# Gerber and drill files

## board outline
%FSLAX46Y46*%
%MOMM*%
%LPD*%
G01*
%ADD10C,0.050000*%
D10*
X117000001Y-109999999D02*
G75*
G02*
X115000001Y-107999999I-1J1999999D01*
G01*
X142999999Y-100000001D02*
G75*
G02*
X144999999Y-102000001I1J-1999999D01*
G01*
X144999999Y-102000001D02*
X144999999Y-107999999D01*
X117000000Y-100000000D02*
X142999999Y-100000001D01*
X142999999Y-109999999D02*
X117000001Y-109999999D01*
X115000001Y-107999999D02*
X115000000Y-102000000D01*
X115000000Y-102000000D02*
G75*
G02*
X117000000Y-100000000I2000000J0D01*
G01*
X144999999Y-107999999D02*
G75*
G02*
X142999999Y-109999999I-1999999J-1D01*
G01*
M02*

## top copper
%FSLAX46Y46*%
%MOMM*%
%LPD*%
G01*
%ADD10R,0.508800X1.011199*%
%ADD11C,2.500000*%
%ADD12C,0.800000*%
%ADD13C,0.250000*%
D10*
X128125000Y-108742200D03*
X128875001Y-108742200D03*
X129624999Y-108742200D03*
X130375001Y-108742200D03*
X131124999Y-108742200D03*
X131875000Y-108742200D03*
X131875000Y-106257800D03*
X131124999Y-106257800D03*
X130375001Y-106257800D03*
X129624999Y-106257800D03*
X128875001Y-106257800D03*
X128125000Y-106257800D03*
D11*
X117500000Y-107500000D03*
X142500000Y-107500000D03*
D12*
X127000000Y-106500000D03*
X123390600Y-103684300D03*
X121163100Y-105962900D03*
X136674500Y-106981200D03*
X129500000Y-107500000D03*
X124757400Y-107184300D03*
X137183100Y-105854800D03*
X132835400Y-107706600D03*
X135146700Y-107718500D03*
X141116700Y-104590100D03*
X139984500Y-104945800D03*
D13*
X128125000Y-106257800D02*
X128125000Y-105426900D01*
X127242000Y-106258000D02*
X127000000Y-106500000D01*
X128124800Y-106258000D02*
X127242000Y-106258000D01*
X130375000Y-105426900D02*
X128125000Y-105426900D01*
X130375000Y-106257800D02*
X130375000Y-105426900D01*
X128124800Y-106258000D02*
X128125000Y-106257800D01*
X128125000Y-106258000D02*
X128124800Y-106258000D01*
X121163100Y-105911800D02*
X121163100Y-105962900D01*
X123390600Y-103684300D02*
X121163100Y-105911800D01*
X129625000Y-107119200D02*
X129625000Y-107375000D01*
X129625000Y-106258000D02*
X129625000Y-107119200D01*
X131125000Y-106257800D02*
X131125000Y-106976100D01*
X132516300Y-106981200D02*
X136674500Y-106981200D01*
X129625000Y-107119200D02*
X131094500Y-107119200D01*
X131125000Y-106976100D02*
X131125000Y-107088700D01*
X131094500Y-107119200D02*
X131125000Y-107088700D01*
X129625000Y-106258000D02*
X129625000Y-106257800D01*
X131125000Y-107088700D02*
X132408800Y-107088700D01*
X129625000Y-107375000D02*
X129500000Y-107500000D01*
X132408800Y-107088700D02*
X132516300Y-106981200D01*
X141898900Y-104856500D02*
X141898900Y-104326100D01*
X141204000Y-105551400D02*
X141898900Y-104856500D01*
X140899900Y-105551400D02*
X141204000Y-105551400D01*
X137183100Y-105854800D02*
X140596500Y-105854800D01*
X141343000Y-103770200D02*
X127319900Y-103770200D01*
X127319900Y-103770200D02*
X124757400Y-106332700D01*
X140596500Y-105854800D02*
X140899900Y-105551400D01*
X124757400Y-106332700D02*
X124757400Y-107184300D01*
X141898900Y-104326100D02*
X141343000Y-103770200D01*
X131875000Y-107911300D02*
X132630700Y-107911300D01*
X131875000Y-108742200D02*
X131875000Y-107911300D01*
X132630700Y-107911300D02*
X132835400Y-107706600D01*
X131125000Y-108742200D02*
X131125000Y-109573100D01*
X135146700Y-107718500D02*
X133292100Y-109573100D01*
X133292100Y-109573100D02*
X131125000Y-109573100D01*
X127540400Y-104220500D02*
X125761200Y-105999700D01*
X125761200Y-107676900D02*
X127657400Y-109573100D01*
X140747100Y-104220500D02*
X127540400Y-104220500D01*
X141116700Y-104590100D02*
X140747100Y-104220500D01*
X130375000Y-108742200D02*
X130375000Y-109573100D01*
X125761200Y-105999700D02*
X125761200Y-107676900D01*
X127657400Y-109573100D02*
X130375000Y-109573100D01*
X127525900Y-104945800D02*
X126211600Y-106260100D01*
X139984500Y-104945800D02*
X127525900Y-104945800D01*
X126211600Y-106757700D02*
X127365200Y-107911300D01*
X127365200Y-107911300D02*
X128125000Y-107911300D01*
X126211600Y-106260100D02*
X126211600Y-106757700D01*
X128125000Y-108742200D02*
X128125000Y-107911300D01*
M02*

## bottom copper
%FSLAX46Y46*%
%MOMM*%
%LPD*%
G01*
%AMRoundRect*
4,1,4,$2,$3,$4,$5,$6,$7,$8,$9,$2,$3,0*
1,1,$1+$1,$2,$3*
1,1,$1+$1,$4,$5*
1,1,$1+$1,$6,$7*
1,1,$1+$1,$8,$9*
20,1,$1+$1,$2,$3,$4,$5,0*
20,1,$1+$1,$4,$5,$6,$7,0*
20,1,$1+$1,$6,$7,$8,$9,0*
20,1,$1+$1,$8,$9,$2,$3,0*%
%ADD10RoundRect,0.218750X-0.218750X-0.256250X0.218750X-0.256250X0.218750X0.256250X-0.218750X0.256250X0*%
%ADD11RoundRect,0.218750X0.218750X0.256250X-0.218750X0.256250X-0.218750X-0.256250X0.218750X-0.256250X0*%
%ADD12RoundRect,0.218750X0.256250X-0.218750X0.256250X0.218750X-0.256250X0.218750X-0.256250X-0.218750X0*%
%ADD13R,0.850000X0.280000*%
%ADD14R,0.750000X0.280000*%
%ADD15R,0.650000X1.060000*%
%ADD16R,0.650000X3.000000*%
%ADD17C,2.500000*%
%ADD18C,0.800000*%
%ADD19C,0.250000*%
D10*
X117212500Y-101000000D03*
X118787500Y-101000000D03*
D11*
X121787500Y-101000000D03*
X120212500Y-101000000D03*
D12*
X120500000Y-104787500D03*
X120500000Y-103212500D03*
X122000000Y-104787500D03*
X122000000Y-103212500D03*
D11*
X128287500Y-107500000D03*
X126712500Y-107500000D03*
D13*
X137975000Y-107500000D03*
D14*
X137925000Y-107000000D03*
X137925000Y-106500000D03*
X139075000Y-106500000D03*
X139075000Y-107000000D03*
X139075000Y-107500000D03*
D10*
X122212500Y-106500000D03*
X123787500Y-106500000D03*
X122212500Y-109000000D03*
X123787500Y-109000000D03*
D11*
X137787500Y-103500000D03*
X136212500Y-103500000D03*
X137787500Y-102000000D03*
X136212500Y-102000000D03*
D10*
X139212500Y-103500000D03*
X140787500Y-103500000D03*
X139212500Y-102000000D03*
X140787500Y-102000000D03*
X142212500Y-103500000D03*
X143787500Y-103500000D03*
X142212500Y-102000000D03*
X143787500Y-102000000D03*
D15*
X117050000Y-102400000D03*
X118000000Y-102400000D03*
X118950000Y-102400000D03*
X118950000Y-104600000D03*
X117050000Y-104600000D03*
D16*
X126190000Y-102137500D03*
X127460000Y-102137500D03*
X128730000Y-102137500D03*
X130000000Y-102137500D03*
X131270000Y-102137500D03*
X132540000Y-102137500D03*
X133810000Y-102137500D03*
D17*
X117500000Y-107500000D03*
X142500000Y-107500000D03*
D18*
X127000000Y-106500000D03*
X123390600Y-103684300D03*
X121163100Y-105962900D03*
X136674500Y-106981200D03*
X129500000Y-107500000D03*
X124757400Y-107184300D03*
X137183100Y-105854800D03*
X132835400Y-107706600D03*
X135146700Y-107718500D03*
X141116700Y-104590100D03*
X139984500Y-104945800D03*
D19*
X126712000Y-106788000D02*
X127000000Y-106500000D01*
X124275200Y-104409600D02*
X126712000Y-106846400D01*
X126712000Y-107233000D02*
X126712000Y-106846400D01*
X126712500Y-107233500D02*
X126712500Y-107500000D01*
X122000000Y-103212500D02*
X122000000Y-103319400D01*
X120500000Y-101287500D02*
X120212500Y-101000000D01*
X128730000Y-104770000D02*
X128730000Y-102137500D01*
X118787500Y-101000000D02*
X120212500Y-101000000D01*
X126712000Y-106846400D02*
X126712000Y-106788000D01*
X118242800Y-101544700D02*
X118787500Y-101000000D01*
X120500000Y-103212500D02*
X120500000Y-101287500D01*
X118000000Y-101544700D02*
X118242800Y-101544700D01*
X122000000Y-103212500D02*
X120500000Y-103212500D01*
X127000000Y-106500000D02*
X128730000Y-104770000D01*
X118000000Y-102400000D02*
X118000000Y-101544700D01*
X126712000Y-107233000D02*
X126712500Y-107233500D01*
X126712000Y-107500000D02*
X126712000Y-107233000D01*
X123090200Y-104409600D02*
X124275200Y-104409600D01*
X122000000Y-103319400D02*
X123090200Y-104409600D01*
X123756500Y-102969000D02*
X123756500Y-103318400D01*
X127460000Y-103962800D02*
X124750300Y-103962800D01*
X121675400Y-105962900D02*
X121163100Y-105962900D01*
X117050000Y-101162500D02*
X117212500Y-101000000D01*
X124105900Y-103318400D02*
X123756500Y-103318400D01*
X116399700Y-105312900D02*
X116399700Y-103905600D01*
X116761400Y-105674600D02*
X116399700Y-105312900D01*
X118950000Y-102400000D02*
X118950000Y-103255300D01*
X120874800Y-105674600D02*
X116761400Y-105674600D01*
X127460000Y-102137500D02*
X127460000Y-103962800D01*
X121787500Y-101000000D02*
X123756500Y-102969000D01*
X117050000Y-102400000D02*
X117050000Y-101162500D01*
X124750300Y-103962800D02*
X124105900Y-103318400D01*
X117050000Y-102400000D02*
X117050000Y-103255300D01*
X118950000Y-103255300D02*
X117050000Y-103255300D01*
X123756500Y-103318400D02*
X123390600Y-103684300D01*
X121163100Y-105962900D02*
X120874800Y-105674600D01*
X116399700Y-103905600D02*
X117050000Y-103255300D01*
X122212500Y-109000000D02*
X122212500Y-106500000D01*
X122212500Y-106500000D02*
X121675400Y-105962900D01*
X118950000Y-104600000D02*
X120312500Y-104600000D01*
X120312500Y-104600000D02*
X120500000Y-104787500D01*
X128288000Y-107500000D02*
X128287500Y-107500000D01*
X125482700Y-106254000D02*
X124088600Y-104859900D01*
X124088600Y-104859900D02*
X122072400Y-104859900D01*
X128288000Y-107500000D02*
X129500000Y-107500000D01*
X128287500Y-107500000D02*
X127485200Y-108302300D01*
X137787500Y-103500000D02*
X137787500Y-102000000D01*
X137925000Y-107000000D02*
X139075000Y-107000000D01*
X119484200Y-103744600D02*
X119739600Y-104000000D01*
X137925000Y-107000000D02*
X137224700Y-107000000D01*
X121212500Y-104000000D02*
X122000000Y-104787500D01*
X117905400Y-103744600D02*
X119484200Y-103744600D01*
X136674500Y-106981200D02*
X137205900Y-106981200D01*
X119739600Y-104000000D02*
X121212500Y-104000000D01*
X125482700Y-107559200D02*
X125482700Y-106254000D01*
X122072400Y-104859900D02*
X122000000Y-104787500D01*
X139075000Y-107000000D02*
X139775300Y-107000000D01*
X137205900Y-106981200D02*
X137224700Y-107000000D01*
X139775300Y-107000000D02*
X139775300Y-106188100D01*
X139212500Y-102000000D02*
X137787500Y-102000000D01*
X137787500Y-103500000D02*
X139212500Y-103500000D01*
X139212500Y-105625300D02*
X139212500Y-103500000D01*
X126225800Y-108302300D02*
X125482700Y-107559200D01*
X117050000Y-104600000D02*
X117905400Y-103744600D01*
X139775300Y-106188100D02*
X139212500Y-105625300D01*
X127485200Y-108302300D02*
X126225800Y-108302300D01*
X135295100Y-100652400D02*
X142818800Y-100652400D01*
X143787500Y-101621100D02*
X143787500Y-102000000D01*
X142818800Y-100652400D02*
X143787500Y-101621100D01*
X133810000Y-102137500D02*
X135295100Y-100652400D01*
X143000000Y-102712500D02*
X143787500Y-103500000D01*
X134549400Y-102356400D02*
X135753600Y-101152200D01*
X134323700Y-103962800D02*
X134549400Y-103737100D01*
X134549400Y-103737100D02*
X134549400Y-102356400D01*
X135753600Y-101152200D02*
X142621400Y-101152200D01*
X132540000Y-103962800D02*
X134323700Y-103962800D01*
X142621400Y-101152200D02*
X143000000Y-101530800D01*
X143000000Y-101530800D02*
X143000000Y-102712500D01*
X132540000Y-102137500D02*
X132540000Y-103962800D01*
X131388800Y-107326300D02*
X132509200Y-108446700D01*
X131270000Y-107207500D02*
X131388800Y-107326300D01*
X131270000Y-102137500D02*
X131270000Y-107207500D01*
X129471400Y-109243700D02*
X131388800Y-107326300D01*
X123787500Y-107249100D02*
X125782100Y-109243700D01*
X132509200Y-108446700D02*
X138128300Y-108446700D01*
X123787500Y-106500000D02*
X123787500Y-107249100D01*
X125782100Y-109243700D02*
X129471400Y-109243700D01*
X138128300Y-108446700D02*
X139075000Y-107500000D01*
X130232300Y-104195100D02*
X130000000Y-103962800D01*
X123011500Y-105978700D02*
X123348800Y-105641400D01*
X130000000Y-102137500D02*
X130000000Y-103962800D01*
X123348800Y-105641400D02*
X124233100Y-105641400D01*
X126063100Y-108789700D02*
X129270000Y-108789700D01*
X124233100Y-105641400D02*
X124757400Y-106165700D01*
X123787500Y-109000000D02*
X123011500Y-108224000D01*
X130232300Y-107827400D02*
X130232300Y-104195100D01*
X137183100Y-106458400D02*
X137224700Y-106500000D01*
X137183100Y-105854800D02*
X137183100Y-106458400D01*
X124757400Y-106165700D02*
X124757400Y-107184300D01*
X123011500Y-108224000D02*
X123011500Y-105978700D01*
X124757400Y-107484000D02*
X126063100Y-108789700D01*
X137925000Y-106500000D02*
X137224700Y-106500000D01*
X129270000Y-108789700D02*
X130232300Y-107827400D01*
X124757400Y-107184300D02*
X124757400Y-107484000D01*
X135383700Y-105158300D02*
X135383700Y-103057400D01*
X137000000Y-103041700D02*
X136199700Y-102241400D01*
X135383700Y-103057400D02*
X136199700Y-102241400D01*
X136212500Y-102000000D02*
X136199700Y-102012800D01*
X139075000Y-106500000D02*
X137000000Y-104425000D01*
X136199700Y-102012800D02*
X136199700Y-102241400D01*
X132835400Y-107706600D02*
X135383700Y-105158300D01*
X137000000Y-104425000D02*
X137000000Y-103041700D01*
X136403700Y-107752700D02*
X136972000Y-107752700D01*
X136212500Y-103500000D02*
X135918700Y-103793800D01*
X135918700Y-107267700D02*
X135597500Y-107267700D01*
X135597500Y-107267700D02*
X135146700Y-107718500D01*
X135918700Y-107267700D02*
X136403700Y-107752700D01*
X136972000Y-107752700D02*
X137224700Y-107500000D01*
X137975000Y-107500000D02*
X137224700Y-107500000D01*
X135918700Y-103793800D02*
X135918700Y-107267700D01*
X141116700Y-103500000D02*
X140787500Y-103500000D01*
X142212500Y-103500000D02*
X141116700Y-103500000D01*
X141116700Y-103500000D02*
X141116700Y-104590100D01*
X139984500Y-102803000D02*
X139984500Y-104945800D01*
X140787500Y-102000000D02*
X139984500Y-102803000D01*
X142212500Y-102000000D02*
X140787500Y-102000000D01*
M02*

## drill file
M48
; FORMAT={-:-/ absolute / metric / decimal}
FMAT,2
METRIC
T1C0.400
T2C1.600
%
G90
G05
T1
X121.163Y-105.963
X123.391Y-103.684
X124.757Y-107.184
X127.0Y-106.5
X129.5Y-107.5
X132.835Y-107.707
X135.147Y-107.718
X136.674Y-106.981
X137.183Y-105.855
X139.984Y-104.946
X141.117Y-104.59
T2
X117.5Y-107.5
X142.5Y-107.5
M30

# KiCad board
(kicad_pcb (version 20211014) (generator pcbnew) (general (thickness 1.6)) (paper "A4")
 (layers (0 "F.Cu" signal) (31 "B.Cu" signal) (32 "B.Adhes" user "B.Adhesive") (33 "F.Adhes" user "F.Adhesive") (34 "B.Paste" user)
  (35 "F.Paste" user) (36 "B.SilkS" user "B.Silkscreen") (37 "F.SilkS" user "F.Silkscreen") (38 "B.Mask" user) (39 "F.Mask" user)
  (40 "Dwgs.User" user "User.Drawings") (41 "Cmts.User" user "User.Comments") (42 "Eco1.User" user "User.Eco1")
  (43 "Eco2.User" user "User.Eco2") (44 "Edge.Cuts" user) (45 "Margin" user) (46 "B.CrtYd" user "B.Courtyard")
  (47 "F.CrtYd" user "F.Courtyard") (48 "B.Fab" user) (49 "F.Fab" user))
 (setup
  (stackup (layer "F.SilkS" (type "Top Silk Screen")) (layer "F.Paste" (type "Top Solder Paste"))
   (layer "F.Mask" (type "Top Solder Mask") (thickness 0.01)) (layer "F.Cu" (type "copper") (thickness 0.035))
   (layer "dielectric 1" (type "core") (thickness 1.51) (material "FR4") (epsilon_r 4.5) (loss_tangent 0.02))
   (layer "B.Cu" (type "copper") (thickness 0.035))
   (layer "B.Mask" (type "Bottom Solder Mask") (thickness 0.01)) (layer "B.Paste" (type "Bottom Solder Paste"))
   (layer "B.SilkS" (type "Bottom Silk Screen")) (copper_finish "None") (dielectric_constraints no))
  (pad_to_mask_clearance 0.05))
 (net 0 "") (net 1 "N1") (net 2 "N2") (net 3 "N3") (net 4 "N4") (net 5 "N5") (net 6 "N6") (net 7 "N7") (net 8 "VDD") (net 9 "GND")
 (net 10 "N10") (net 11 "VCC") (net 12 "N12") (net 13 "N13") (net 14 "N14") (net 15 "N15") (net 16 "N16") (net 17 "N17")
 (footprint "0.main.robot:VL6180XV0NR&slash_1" (layer "F.Cu") (at 130 107.5 90)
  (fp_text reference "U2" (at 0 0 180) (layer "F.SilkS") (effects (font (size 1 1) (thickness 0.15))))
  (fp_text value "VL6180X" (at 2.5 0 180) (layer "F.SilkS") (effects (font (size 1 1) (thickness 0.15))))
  (pad "1" smd rect locked (at -1.2422 -1.875 90) (size 1.011199 0.5088) (layers "F.Cu" "F.Paste" "F.Mask") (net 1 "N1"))
  (pad "2" smd rect locked (at -1.2422 -1.124999 90) (size 1.011199 0.5088) (layers "F.Cu" "F.Paste" "F.Mask") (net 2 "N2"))
  (pad "3" smd rect locked (at -1.2422 -0.375001 90) (size 1.011199 0.5088) (layers "F.Cu" "F.Paste" "F.Mask") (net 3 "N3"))
  (pad "4" smd rect locked (at -1.2422 0.375001 90) (size 1.011199 0.5088) (layers "F.Cu" "F.Paste" "F.Mask") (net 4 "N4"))
  (pad "5" smd rect locked (at -1.2422 1.124999 90) (size 1.011199 0.5088) (layers "F.Cu" "F.Paste" "F.Mask") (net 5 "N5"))
  (pad "6" smd rect locked (at -1.2422 1.875 90) (size 1.011199 0.5088) (layers "F.Cu" "F.Paste" "F.Mask") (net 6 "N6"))
  (pad "7" smd rect locked (at 1.2422 1.875 90) (size 1.011199 0.5088) (layers "F.Cu" "F.Paste" "F.Mask") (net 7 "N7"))
  (pad "8" smd rect locked (at 1.2422 1.124999 90) (size 1.011199 0.5088) (layers "F.Cu" "F.Paste" "F.Mask") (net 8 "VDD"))
  (pad "9" smd rect locked (at 1.2422 0.375001 90) (size 1.011199 0.5088) (layers "F.Cu" "F.Paste" "F.Mask") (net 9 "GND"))
  (pad "10" smd rect locked (at 1.2422 -0.375001 90) (size 1.011199 0.5088) (layers "F.Cu" "F.Paste" "F.Mask") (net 8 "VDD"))
  (pad "11" smd rect locked (at 1.2422 -1.124999 90) (size 1.011199 0.5088) (layers "F.Cu" "F.Paste" "F.Mask") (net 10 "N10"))
  (pad "12" smd rect locked (at 1.2422 -1.875 90) (size 1.011199 0.5088) (layers "F.Cu" "F.Paste" "F.Mask") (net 9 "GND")))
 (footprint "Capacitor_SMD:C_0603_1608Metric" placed (layer "B.Cu") (at 118 101)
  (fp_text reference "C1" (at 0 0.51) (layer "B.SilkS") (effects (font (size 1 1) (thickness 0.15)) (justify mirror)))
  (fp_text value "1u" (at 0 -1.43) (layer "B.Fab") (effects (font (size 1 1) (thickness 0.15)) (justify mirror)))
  (pad "1" smd roundrect locked (at -0.7875 0) (size 0.875 0.95) (layers "B.Cu" "B.Paste" "B.Mask") (roundrect_rratio 0.25) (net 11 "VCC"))
  (pad "2" smd roundrect locked (at 0.7875 0) (size 0.875 0.95) (layers "B.Cu" "B.Paste" "B.Mask") (roundrect_rratio 0.25) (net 9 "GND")))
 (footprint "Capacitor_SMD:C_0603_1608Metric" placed (layer "B.Cu") (at 121 101 180)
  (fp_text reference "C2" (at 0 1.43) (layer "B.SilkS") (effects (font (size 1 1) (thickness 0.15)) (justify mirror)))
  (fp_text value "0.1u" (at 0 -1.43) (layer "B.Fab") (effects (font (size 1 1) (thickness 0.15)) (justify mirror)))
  (pad "1" smd roundrect locked (at -0.7875 0 180) (size 0.875 0.95) (layers "B.Cu" "B.Paste" "B.Mask") (roundrect_rratio 0.25)
   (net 11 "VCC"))
  (pad "2" smd roundrect locked (at 0.7875 0 180) (size 0.875 0.95) (layers "B.Cu" "B.Paste" "B.Mask") (roundrect_rratio 0.25) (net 9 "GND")))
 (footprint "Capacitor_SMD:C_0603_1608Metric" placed (layer "B.Cu") (at 120.5 104 90)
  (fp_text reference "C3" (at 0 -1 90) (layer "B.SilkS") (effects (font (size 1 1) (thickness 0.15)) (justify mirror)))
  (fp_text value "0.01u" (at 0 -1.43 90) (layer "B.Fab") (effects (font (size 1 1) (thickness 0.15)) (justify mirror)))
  (pad "1" smd roundrect locked (at -0.7875 0 90) (size 0.875 0.95) (layers "B.Cu" "B.Paste" "B.Mask") (roundrect_rratio 0.25)
   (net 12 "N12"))
  (pad "2" smd roundrect locked (at 0.7875 0 90) (size 0.875 0.95) (layers "B.Cu" "B.Paste" "B.Mask") (roundrect_rratio 0.25) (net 9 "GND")))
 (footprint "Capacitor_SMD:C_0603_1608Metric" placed (layer "B.Cu") (at 122 104 90)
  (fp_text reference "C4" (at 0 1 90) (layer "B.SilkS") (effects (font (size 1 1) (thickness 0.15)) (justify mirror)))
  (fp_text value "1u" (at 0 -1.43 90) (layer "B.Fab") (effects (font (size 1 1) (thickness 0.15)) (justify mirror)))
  (pad "1" smd roundrect locked (at -0.7875 0 90) (size 0.875 0.95) (layers "B.Cu" "B.Paste" "B.Mask") (roundrect_rratio 0.25) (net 8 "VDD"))
  (pad "2" smd roundrect locked (at 0.7875 0 90) (size 0.875 0.95) (layers "B.Cu" "B.Paste" "B.Mask") (roundrect_rratio 0.25) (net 9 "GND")))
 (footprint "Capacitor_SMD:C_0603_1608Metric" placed (layer "B.Cu") (at 127.5 107.5 180)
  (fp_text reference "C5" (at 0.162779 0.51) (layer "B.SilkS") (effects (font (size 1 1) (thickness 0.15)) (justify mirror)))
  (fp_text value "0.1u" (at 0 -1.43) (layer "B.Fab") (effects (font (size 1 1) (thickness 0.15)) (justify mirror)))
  (pad "1" smd roundrect locked (at -0.7875 0 180) (size 0.875 0.95) (layers "B.Cu" "B.Paste" "B.Mask") (roundrect_rratio 0.25)
   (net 8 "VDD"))
  (pad "2" smd roundrect locked (at 0.7875 0 180) (size 0.875 0.95) (layers "B.Cu" "B.Paste" "B.Mask") (roundrect_rratio 0.25) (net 9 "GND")))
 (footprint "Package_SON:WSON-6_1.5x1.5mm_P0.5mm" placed (layer "B.Cu") (at 138.5 107)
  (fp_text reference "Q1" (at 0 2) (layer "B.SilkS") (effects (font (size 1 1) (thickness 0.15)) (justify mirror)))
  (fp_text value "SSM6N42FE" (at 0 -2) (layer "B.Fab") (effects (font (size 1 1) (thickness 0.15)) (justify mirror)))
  (pad "1" smd rect locked (at -0.525 0.5 90) (size 0.28 0.85) (layers "B.Cu" "B.Paste" "B.Mask") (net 5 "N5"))
  (pad "2" smd rect locked (at -0.575 0 90) (size 0.28 0.75) (layers "B.Cu" "B.Paste" "B.Mask") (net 8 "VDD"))
  (pad "3" smd rect locked (at -0.575 -0.5 90) (size 0.28 0.75) (layers "B.Cu" "B.Paste" "B.Mask") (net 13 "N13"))
  (pad "4" smd rect locked (at 0.575 -0.5 90) (size 0.28 0.75) (layers "B.Cu" "B.Paste" "B.Mask") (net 6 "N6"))
  (pad "5" smd rect locked (at 0.575 0 90) (size 0.28 0.75) (layers "B.Cu" "B.Paste" "B.Mask") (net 8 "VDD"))
  (pad "6" smd rect locked (at 0.575 0.5 90) (size 0.28 0.75) (layers "B.Cu" "B.Paste" "B.Mask") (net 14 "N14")))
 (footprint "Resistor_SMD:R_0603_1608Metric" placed (layer "B.Cu") (at 123 106.5)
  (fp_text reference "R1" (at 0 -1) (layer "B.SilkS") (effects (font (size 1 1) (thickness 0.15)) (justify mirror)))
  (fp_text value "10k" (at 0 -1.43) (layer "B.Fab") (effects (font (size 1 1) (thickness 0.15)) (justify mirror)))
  (pad "1" smd roundrect locked (at -0.7875 0) (size 0.875 0.95) (layers "B.Cu" "B.Paste" "B.Mask") (roundrect_rratio 0.25) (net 11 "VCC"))
  (pad "2" smd roundrect locked (at 0.7875 0) (size 0.875 0.95) (layers "B.Cu" "B.Paste" "B.Mask") (roundrect_rratio 0.25) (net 14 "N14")))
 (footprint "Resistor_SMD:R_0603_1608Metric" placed (layer "B.Cu") (at 123 109)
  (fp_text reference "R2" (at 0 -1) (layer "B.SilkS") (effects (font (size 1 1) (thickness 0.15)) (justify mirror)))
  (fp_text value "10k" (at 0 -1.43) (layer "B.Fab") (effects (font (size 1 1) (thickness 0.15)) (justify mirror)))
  (pad "1" smd roundrect locked (at -0.7875 0) (size 0.875 0.95) (layers "B.Cu" "B.Paste" "B.Mask") (roundrect_rratio 0.25) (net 11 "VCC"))
  (pad "2" smd roundrect locked (at 0.7875 0) (size 0.875 0.95) (layers "B.Cu" "B.Paste" "B.Mask") (roundrect_rratio 0.25) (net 13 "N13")))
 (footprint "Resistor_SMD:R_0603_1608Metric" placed (layer "B.Cu") (at 137 103.5 180)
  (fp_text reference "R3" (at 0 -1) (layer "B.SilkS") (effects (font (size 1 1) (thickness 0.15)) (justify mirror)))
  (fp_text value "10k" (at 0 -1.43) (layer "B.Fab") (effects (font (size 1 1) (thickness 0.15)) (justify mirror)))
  (pad "1" smd roundrect locked (at -0.7875 0 180) (size 0.875 0.95) (layers "B.Cu" "B.Paste" "B.Mask") (roundrect_rratio 0.25)
   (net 8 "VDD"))
  (pad "2" smd roundrect locked (at 0.7875 0 180) (size 0.875 0.95) (layers "B.Cu" "B.Paste" "B.Mask") (roundrect_rratio 0.25) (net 5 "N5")))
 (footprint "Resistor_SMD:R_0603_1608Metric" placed (layer "B.Cu") (at 137 102 180)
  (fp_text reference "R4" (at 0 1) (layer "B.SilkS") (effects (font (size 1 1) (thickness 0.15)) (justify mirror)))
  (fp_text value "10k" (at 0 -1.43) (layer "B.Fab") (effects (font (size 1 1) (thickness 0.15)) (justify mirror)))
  (pad "1" smd roundrect locked (at -0.7875 0 180) (size 0.875 0.95) (layers "B.Cu" "B.Paste" "B.Mask") (roundrect_rratio 0.25)
   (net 8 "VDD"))
  (pad "2" smd roundrect locked (at 0.7875 0 180) (size 0.875 0.95) (layers "B.Cu" "B.Paste" "B.Mask") (roundrect_rratio 0.25) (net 6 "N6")))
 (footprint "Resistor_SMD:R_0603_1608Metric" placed (layer "B.Cu") (at 140 103.5)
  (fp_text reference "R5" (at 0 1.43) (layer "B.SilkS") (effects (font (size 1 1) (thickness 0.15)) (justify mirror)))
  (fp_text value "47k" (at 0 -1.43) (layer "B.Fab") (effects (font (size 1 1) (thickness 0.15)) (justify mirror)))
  (pad "1" smd roundrect locked (at -0.7875 0) (size 0.875 0.95) (layers "B.Cu" "B.Paste" "B.Mask") (roundrect_rratio 0.25) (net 8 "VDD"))
  (pad "2" smd roundrect locked (at 0.7875 0) (size 0.875 0.95) (layers "B.Cu" "B.Paste" "B.Mask") (roundrect_rratio 0.25) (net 4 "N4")))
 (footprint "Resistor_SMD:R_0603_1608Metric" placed (layer "B.Cu") (at 140 102)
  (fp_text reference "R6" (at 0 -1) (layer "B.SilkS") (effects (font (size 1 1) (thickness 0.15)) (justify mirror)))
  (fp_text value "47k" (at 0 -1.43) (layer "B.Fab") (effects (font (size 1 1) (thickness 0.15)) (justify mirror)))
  (pad "1" smd roundrect locked (at -0.7875 0) (size 0.875 0.95) (layers "B.Cu" "B.Paste" "B.Mask") (roundrect_rratio 0.25) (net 8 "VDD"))
  (pad "2" smd roundrect locked (at 0.7875 0) (size 0.875 0.95) (layers "B.Cu" "B.Paste" "B.Mask") (roundrect_rratio 0.25) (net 1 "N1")))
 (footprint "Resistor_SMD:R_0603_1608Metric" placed (layer "B.Cu") (at 143 103.5)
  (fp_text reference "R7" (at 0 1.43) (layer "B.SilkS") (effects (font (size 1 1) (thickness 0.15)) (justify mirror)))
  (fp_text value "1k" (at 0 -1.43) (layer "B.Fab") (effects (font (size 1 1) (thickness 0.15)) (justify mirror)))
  (pad "1" smd roundrect locked (at -0.7875 0) (size 0.875 0.95) (layers "B.Cu" "B.Paste" "B.Mask") (roundrect_rratio 0.25) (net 4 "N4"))
  (pad "2" smd roundrect locked (at 0.7875 0) (size 0.875 0.95) (layers "B.Cu" "B.Paste" "B.Mask") (roundrect_rratio 0.25) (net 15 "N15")))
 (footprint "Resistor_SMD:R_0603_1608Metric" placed (layer "B.Cu") (at 143 102)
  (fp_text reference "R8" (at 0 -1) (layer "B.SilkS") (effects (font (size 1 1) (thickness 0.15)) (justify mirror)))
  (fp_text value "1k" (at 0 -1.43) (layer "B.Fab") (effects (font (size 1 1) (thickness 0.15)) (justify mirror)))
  (pad "1" smd roundrect locked (at -0.7875 0) (size 0.875 0.95) (layers "B.Cu" "B.Paste" "B.Mask") (roundrect_rratio 0.25) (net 1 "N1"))
  (pad "2" smd roundrect locked (at 0.7875 0) (size 0.875 0.95) (layers "B.Cu" "B.Paste" "B.Mask") (roundrect_rratio 0.25) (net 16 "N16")))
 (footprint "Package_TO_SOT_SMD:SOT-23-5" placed (layer "B.Cu") (at 118 103.5 -90)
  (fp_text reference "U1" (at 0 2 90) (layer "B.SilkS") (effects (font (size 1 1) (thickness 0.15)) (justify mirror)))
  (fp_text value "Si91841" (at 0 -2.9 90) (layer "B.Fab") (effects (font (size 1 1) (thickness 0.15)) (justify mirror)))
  (pad "1" smd rect locked (at -1.1 0.95 270) (size 1.06 0.65) (layers "B.Cu" "B.Paste" "B.Mask") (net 11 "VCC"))
  (pad "2" smd rect locked (at -1.1 0 270) (size 1.06 0.65) (layers "B.Cu" "B.Paste" "B.Mask") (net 9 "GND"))
  (pad "3" smd rect locked (at -1.1 -0.95 270) (size 1.06 0.65) (layers "B.Cu" "B.Paste" "B.Mask") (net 11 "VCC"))
  (pad "4" smd rect locked (at 1.1 -0.95 270) (size 1.06 0.65) (layers "B.Cu" "B.Paste" "B.Mask") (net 12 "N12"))
  (pad "5" smd rect locked (at 1.1 0.95 270) (size 1.06 0.65) (layers "B.Cu" "B.Paste" "B.Mask") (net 8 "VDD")))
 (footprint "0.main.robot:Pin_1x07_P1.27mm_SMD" (layer "B.Cu") (at 130 103.6375 -90)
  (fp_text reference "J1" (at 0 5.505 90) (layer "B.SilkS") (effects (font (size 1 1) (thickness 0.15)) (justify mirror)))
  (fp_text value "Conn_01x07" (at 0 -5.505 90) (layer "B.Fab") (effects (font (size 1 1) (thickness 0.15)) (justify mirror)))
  (pad "1" smd rect locked (at -1.5 3.81 270) (size 3 0.65) (layers "B.Cu" "B.Paste" "B.Mask") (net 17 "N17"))
  (pad "2" smd rect locked (at -1.5 2.54 270) (size 3 0.65) (layers "B.Cu" "B.Paste" "B.Mask") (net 11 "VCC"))
  (pad "3" smd rect locked (at -1.5 1.27 270) (size 3 0.65) (layers "B.Cu" "B.Paste" "B.Mask") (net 9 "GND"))
  (pad "4" smd rect locked (at -1.5 0 270) (size 3 0.65) (layers "B.Cu" "B.Paste" "B.Mask") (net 13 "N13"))
  (pad "5" smd rect locked (at -1.5 -1.27 270) (size 3 0.65) (layers "B.Cu" "B.Paste" "B.Mask") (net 14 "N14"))
  (pad "6" smd rect locked (at -1.5 -2.54 270) (size 3 0.65) (layers "B.Cu" "B.Paste" "B.Mask") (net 15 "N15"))
  (pad "7" smd rect locked (at -1.5 -3.81 270) (size 3 0.65) (layers "B.Cu" "B.Paste" "B.Mask") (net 16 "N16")))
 (gr_arc (start 117.000001 109.999999) (mid 115.585787 109.414213) (end 115.000001 107.999999) (layer "Edge.Cuts") (width 0.05))
 (gr_arc (start 142.999999 100.000001) (mid 144.414213 100.585787) (end 144.999999 102.000001) (layer "Edge.Cuts") (width 0.05))
 (gr_line (start 144.999999 102.000001) (end 144.999999 107.999999) (layer "Edge.Cuts") (width 0.05))
 (gr_line (start 117 100) (end 142.999999 100.000001) (layer "Edge.Cuts") (width 0.05))
 (gr_line (start 142.999999 109.999999) (end 117.000001 109.999999) (layer "Edge.Cuts") (width 0.05))
 (gr_line (start 115.000001 107.999999) (end 115 102) (layer "Edge.Cuts") (width 0.05))
 (gr_arc (start 115 102) (mid 115.585786 100.585786) (end 117 100) (layer "Edge.Cuts") (width 0.05))
 (gr_arc (start 144.999999 107.999999) (mid 144.414213 109.414213) (end 142.999999 109.999999) (layer "Edge.Cuts") (width 0.05))
 (via (at 117.5 107.5) (size 2.5) (drill 1.6) (layers "F.Cu" "B.Cu") (free) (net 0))
 (via (at 142.5 107.5) (size 2.5) (drill 1.6) (layers "F.Cu" "B.Cu") (free) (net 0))
 (segment (start 128.125 106.2578) (end 128.125 105.4269) (width 0.25) (layer "F.Cu") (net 9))
 (segment (start 127.242 106.258) (end 127 106.5) (width 0.25) (layer "F.Cu") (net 9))
 (segment (start 128.1248 106.258) (end 127.242 106.258) (width 0.25) (layer "F.Cu") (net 9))
 (segment (start 130.375 105.4269) (end 128.125 105.4269) (width 0.25) (layer "F.Cu") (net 9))
 (segment (start 130.375 106.2578) (end 130.375 105.4269) (width 0.25) (layer "F.Cu") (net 9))
 (segment (start 128.1248 106.258) (end 128.125 106.2578) (width 0.25) (layer "F.Cu") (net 9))
 (segment (start 128.125 106.258) (end 128.1248 106.258) (width 0.25) (layer "F.Cu") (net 9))
 (via (at 127 106.5) (size 0.8) (drill 0.4) (layers "F.Cu" "B.Cu") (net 9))
 (segment (start 126.712 106.788) (end 127 106.5) (width 0.25) (layer "B.Cu") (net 9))
 (segment (start 124.2752 104.4096) (end 126.712 106.8464) (width 0.25) (layer "B.Cu") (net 9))
 (segment (start 126.712 107.233) (end 126.712 106.8464) (width 0.25) (layer "B.Cu") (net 9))
 (segment (start 126.7125 107.2335) (end 126.7125 107.5) (width 0.25) (layer "B.Cu") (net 9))
 (segment (start 122 103.2125) (end 122 103.3194) (width 0.25) (layer "B.Cu") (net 9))
 (segment (start 120.5 101.2875) (end 120.2125 101) (width 0.25) (layer "B.Cu") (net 9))
 (segment (start 128.73 104.77) (end 128.73 102.1375) (width 0.25) (layer "B.Cu") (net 9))
 (segment (start 118.7875 101) (end 120.2125 101) (width 0.25) (layer "B.Cu") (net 9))
 (segment (start 126.712 106.8464) (end 126.712 106.788) (width 0.25) (layer "B.Cu") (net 9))
 (segment (start 118.2428 101.5447) (end 118.7875 101) (width 0.25) (layer "B.Cu") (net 9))
 (segment (start 120.5 103.2125) (end 120.5 101.2875) (width 0.25) (layer "B.Cu") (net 9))
 (segment (start 118 101.5447) (end 118.2428 101.5447) (width 0.25) (layer "B.Cu") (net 9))
 (segment (start 122 103.2125) (end 120.5 103.2125) (width 0.25) (layer "B.Cu") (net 9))
 (segment (start 127 106.5) (end 128.73 104.77) (width 0.25) (layer "B.Cu") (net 9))
 (segment (start 118 102.4) (end 118 101.5447) (width 0.25) (layer "B.Cu") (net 9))
 (segment (start 126.712 107.233) (end 126.7125 107.2335) (width 0.25) (layer "B.Cu") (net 9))
 (segment (start 126.712 107.5) (end 126.712 107.233) (width 0.25) (layer "B.Cu") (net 9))
 (segment (start 123.0902 104.4096) (end 124.2752 104.4096) (width 0.25) (layer "B.Cu") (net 9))
 (segment (start 122 103.3194) (end 123.0902 104.4096) (width 0.25) (layer "B.Cu") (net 9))
 (segment (start 121.1631 105.9118) (end 121.1631 105.9629) (width 0.25) (layer "F.Cu") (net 11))
 (segment (start 123.3906 103.6843) (end 121.1631 105.9118) (width 0.25) (layer "F.Cu") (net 11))
 (via (at 123.3906 103.6843) (size 0.8) (drill 0.4) (layers "F.Cu" "B.Cu") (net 11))
 (via (at 121.1631 105.9629) (size 0.8) (drill 0.4) (layers "F.Cu" "B.Cu") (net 11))
 (segment (start 123.7565 102.969) (end 123.7565 103.3184) (width 0.25) (layer "B.Cu") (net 11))
 (segment (start 127.46 103.9628) (end 124.7503 103.9628) (width 0.25) (layer "B.Cu") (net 11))
 (segment (start 121.6754 105.9629) (end 121.1631 105.9629) (width 0.25) (layer "B.Cu") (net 11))
 (segment (start 117.05 101.1625) (end 117.2125 101) (width 0.25) (layer "B.Cu") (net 11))
 (segment (start 124.1059 103.3184) (end 123.7565 103.3184) (width 0.25) (layer "B.Cu") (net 11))
 (segment (start 116.3997 105.3129) (end 116.3997 103.9056) (width 0.25) (layer "B.Cu") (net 11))
 (segment (start 116.7614 105.6746) (end 116.3997 105.3129) (width 0.25) (layer "B.Cu") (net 11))
 (segment (start 118.95 102.4) (end 118.95 103.2553) (width 0.25) (layer "B.Cu") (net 11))
 (segment (start 120.8748 105.6746) (end 116.7614 105.6746) (width 0.25) (layer "B.Cu") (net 11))
 (segment (start 127.46 102.1375) (end 127.46 103.9628) (width 0.25) (layer "B.Cu") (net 11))
 (segment (start 121.7875 101) (end 123.7565 102.969) (width 0.25) (layer "B.Cu") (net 11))
 (segment (start 117.05 102.4) (end 117.05 101.1625) (width 0.25) (layer "B.Cu") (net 11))
 (segment (start 124.7503 103.9628) (end 124.1059 103.3184) (width 0.25) (layer "B.Cu") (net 11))
 (segment (start 117.05 102.4) (end 117.05 103.2553) (width 0.25) (layer "B.Cu") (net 11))
 (segment (start 118.95 103.2553) (end 117.05 103.2553) (width 0.25) (layer "B.Cu") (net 11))
 (segment (start 123.7565 103.3184) (end 123.3906 103.6843) (width 0.25) (layer "B.Cu") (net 11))
 (segment (start 121.1631 105.9629) (end 120.8748 105.6746) (width 0.25) (layer "B.Cu") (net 11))
 (segment (start 116.3997 103.9056) (end 117.05 103.2553) (width 0.25) (layer "B.Cu") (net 11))
 (segment (start 122.2125 109) (end 122.2125 106.5) (width 0.25) (layer "B.Cu") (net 11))
 (segment (start 122.2125 106.5) (end 121.6754 105.9629) (width 0.25) (layer "B.Cu") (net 11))
 (segment (start 118.95 104.6) (end 120.3125 104.6) (width 0.25) (layer "B.Cu") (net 12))
 (segment (start 120.3125 104.6) (end 120.5 104.7875) (width 0.25) (layer "B.Cu") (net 12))
 (segment (start 129.625 107.1192) (end 129.625 107.375) (width 0.25) (layer "F.Cu") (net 8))
 (segment (start 129.625 106.258) (end 129.625 107.1192) (width 0.25) (layer "F.Cu") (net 8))
 (segment (start 131.125 106.2578) (end 131.125 106.9761) (width 0.25) (layer "F.Cu") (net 8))
 (segment (start 132.5163 106.9812) (end 136.6745 106.9812) (width 0.25) (layer "F.Cu") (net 8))
 (segment (start 129.625 107.1192) (end 131.0945 107.1192) (width 0.25) (layer "F.Cu") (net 8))
 (segment (start 131.125 106.9761) (end 131.125 107.0887) (width 0.25) (layer "F.Cu") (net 8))
 (segment (start 131.0945 107.1192) (end 131.125 107.0887) (width 0.25) (layer "F.Cu") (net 8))
 (segment (start 129.625 106.258) (end 129.625 106.2578) (width 0.25) (layer "F.Cu") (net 8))
 (segment (start 131.125 107.0887) (end 132.4088 107.0887) (width 0.25) (layer "F.Cu") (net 8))
 (segment (start 129.625 107.375) (end 129.5 107.5) (width 0.25) (layer "F.Cu") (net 8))
 (segment (start 132.4088 107.0887) (end 132.5163 106.9812) (width 0.25) (layer "F.Cu") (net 8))
 (via (at 136.6745 106.9812) (size 0.8) (drill 0.4) (layers "F.Cu" "B.Cu") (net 8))
 (via (at 129.5 107.5) (size 0.8) (drill 0.4) (layers "F.Cu" "B.Cu") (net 8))
 (segment (start 128.288 107.5) (end 128.2875 107.5) (width 0.25) (layer "B.Cu") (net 8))
 (segment (start 125.4827 106.254) (end 124.0886 104.8599) (width 0.25) (layer "B.Cu") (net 8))
 (segment (start 124.0886 104.8599) (end 122.0724 104.8599) (width 0.25) (layer "B.Cu") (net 8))
 (segment (start 128.288 107.5) (end 129.5 107.5) (width 0.25) (layer "B.Cu") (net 8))
 (segment (start 128.2875 107.5) (end 127.4852 108.3023) (width 0.25) (layer "B.Cu") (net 8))
 (segment (start 137.7875 103.5) (end 137.7875 102) (width 0.25) (layer "B.Cu") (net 8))
 (segment (start 137.925 107) (end 139.075 107) (width 0.25) (layer "B.Cu") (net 8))
 (segment (start 119.4842 103.7446) (end 119.7396 104) (width 0.25) (layer "B.Cu") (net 8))
 (segment (start 137.925 107) (end 137.2247 107) (width 0.25) (layer "B.Cu") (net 8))
 (segment (start 121.2125 104) (end 122 104.7875) (width 0.25) (layer "B.Cu") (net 8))
 (segment (start 117.9054 103.7446) (end 119.4842 103.7446) (width 0.25) (layer "B.Cu") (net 8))
 (segment (start 136.6745 106.9812) (end 137.2059 106.9812) (width 0.25) (layer "B.Cu") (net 8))
 (segment (start 119.7396 104) (end 121.2125 104) (width 0.25) (layer "B.Cu") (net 8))
 (segment (start 125.4827 107.5592) (end 125.4827 106.254) (width 0.25) (layer "B.Cu") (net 8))
 (segment (start 122.0724 104.8599) (end 122 104.7875) (width 0.25) (layer "B.Cu") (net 8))
 (segment (start 139.075 107) (end 139.7753 107) (width 0.25) (layer "B.Cu") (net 8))
 (segment (start 137.2059 106.9812) (end 137.2247 107) (width 0.25) (layer "B.Cu") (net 8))
 (segment (start 139.7753 107) (end 139.7753 106.1881) (width 0.25) (layer "B.Cu") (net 8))
 (segment (start 139.2125 102) (end 137.7875 102) (width 0.25) (layer "B.Cu") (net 8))
 (segment (start 137.7875 103.5) (end 139.2125 103.5) (width 0.25) (layer "B.Cu") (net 8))
 (segment (start 139.2125 105.6253) (end 139.2125 103.5) (width 0.25) (layer "B.Cu") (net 8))
 (segment (start 126.2258 108.3023) (end 125.4827 107.5592) (width 0.25) (layer "B.Cu") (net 8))
 (segment (start 117.05 104.6) (end 117.9054 103.7446) (width 0.25) (layer "B.Cu") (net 8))
 (segment (start 139.7753 106.1881) (end 139.2125 105.6253) (width 0.25) (layer "B.Cu") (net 8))
 (segment (start 127.4852 108.3023) (end 126.2258 108.3023) (width 0.25) (layer "B.Cu") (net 8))
 (segment (start 135.2951 100.6524) (end 142.8188 100.6524) (width 0.25) (layer "B.Cu") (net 16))
 (segment (start 143.7875 101.6211) (end 143.7875 102) (width 0.25) (layer "B.Cu") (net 16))
 (segment (start 142.8188 100.6524) (end 143.7875 101.6211) (width 0.25) (layer "B.Cu") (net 16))
 (segment (start 133.81 102.1375) (end 135.2951 100.6524) (width 0.25) (layer "B.Cu") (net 16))
 (segment (start 143 102.7125) (end 143.7875 103.5) (width 0.25) (layer "B.Cu") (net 15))
 (segment (start 134.5494 102.3564) (end 135.7536 101.1522) (width 0.25) (layer "B.Cu") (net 15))
 (segment (start 134.3237 103.9628) (end 134.5494 103.7371) (width 0.25) (layer "B.Cu") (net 15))
 (segment (start 134.5494 103.7371) (end 134.5494 102.3564) (width 0.25) (layer "B.Cu") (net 15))
 (segment (start 135.7536 101.1522) (end 142.6214 101.1522) (width 0.25) (layer "B.Cu") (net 15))
 (segment (start 132.54 103.9628) (end 134.3237 103.9628) (width 0.25) (layer "B.Cu") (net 15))
 (segment (start 142.6214 101.1522) (end 143 101.5308) (width 0.25) (layer "B.Cu") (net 15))
 (segment (start 143 101.5308) (end 143 102.7125) (width 0.25) (layer "B.Cu") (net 15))
 (segment (start 132.54 102.1375) (end 132.54 103.9628) (width 0.25) (layer "B.Cu") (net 15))
 (segment (start 131.3888 107.3263) (end 132.5092 108.4467) (width 0.25) (layer "B.Cu") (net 14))
 (segment (start 131.27 107.2075) (end 131.3888 107.3263) (width 0.25) (layer "B.Cu") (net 14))
 (segment (start 131.27 102.1375) (end 131.27 107.2075) (width 0.25) (layer "B.Cu") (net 14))
 (segment (start 129.4714 109.2437) (end 131.3888 107.3263) (width 0.25) (layer "B.Cu") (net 14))
 (segment (start 123.7875 107.2491) (end 125.7821 109.2437) (width 0.25) (layer "B.Cu") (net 14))
 (segment (start 132.5092 108.4467) (end 138.1283 108.4467) (width 0.25) (layer "B.Cu") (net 14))
 (segment (start 123.7875 106.5) (end 123.7875 107.2491) (width 0.25) (layer "B.Cu") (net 14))
 (segment (start 125.7821 109.2437) (end 129.4714 109.2437) (width 0.25) (layer "B.Cu") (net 14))
 (segment (start 138.1283 108.4467) (end 139.075 107.5) (width 0.25) (layer "B.Cu") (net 14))
 (segment (start 141.8989 104.8565) (end 141.8989 104.3261) (width 0.25) (layer "F.Cu") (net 13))
 (segment (start 141.204 105.5514) (end 141.8989 104.8565) (width 0.25) (layer "F.Cu") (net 13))
 (segment (start 140.8999 105.5514) (end 141.204 105.5514) (width 0.25) (layer "F.Cu") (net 13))
 (segment (start 137.1831 105.8548) (end 140.5965 105.8548) (width 0.25) (layer "F.Cu") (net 13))
 (segment (start 141.343 103.7702) (end 127.3199 103.7702) (width 0.25) (layer "F.Cu") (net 13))
 (segment (start 127.3199 103.7702) (end 124.7574 106.3327) (width 0.25) (layer "F.Cu") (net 13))
 (segment (start 140.5965 105.8548) (end 140.8999 105.5514) (width 0.25) (layer "F.Cu") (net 13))
 (segment (start 124.7574 106.3327) (end 124.7574 107.1843) (width 0.25) (layer "F.Cu") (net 13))
 (segment (start 141.8989 104.3261) (end 141.343 103.7702) (width 0.25) (layer "F.Cu") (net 13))
 (via (at 124.7574 107.1843) (size 0.8) (drill 0.4) (layers "F.Cu" "B.Cu") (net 13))
 (via (at 137.1831 105.8548) (size 0.8) (drill 0.4) (layers "F.Cu" "B.Cu") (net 13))
 (segment (start 130.2323 104.1951) (end 130 103.9628) (width 0.25) (layer "B.Cu") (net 13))
 (segment (start 123.0115 105.9787) (end 123.3488 105.6414) (width 0.25) (layer "B.Cu") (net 13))
 (segment (start 130 102.1375) (end 130 103.9628) (width 0.25) (layer "B.Cu") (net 13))
 (segment (start 123.3488 105.6414) (end 124.2331 105.6414) (width 0.25) (layer "B.Cu") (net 13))
 (segment (start 126.0631 108.7897) (end 129.27 108.7897) (width 0.25) (layer "B.Cu") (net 13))
 (segment (start 124.2331 105.6414) (end 124.7574 106.1657) (width 0.25) (layer "B.Cu") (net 13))
 (segment (start 123.7875 109) (end 123.0115 108.224) (width 0.25) (layer "B.Cu") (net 13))
 (segment (start 130.2323 107.8274) (end 130.2323 104.1951) (width 0.25) (layer "B.Cu") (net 13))
 (segment (start 137.1831 106.4584) (end 137.2247 106.5) (width 0.25) (layer "B.Cu") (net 13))
 (segment (start 137.1831 105.8548) (end 137.1831 106.4584) (width 0.25) (layer "B.Cu") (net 13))
 (segment (start 124.7574 106.1657) (end 124.7574 107.1843) (width 0.25) (layer "B.Cu") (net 13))
 (segment (start 123.0115 108.224) (end 123.0115 105.9787) (width 0.25) (layer "B.Cu") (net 13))
 (segment (start 124.7574 107.484) (end 126.0631 108.7897) (width 0.25) (layer "B.Cu") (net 13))
 (segment (start 137.925 106.5) (end 137.2247 106.5) (width 0.25) (layer "B.Cu") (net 13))
 (segment (start 129.27 108.7897) (end 130.2323 107.8274) (width 0.25) (layer "B.Cu") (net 13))
 (segment (start 124.7574 107.1843) (end 124.7574 107.484) (width 0.25) (layer "B.Cu") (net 13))
 (segment (start 131.875 107.9113) (end 132.6307 107.9113) (width 0.25) (layer "F.Cu") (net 6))
 (segment (start 131.875 108.7422) (end 131.875 107.9113) (width 0.25) (layer "F.Cu") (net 6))
 (segment (start 132.6307 107.9113) (end 132.8354 107.7066) (width 0.25) (layer "F.Cu") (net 6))
 (via (at 132.8354 107.7066) (size 0.8) (drill 0.4) (layers "F.Cu" "B.Cu") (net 6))
 (segment (start 135.3837 105.1583) (end 135.3837 103.0574) (width 0.25) (layer "B.Cu") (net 6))
 (segment (start 137 103.0417) (end 136.1997 102.2414) (width 0.25) (layer "B.Cu") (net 6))
 (segment (start 135.3837 103.0574) (end 136.1997 102.2414) (width 0.25) (layer "B.Cu") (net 6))
 (segment (start 136.2125 102) (end 136.1997 102.0128) (width 0.25) (layer "B.Cu") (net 6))
 (segment (start 139.075 106.5) (end 137 104.425) (width 0.25) (layer "B.Cu") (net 6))
 (segment (start 136.1997 102.0128) (end 136.1997 102.2414) (width 0.25) (layer "B.Cu") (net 6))
 (segment (start 132.8354 107.7066) (end 135.3837 105.1583) (width 0.25) (layer "B.Cu") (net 6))
 (segment (start 137 104.425) (end 137 103.0417) (width 0.25) (layer "B.Cu") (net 6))
 (segment (start 131.125 108.7422) (end 131.125 109.5731) (width 0.25) (layer "F.Cu") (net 5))
 (segment (start 135.1467 107.7185) (end 133.2921 109.5731) (width 0.25) (layer "F.Cu") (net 5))
 (segment (start 133.2921 109.5731) (end 131.125 109.5731) (width 0.25) (layer "F.Cu") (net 5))
 (via (at 135.1467 107.7185) (size 0.8) (drill 0.4) (layers "F.Cu" "B.Cu") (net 5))
 (segment (start 136.4037 107.7527) (end 136.972 107.7527) (width 0.25) (layer "B.Cu") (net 5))
 (segment (start 136.2125 103.5) (end 135.9187 103.7938) (width 0.25) (layer "B.Cu") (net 5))
 (segment (start 135.9187 107.2677) (end 135.5975 107.2677) (width 0.25) (layer "B.Cu") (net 5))
 (segment (start 135.5975 107.2677) (end 135.1467 107.7185) (width 0.25) (layer "B.Cu") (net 5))
 (segment (start 135.9187 107.2677) (end 136.4037 107.7527) (width 0.25) (layer "B.Cu") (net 5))
 (segment (start 136.972 107.7527) (end 137.2247 107.5) (width 0.25) (layer "B.Cu") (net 5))
 (segment (start 137.975 107.5) (end 137.2247 107.5) (width 0.25) (layer "B.Cu") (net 5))
 (segment (start 135.9187 103.7938) (end 135.9187 107.2677) (width 0.25) (layer "B.Cu") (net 5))
 (segment (start 127.5404 104.2205) (end 125.7612 105.9997) (width 0.25) (layer "F.Cu") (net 4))
 (segment (start 125.7612 107.6769) (end 127.6574 109.5731) (width 0.25) (layer "F.Cu") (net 4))
 (segment (start 140.7471 104.2205) (end 127.5404 104.2205) (width 0.25) (layer "F.Cu") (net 4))
 (segment (start 141.1167 104.5901) (end 140.7471 104.2205) (width 0.25) (layer "F.Cu") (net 4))
 (segment (start 130.375 108.7422) (end 130.375 109.5731) (width 0.25) (layer "F.Cu") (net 4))
 (segment (start 125.7612 105.9997) (end 125.7612 107.6769) (width 0.25) (layer "F.Cu") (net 4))
 (segment (start 127.6574 109.5731) (end 130.375 109.5731) (width 0.25) (layer "F.Cu") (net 4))
 (via (at 141.1167 104.5901) (size 0.8) (drill 0.4) (layers "F.Cu" "B.Cu") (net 4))
 (segment (start 141.1167 103.5) (end 140.7875 103.5) (width 0.25) (layer "B.Cu") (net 4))
 (segment (start 142.2125 103.5) (end 141.1167 103.5) (width 0.25) (layer "B.Cu") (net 4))
 (segment (start 141.1167 103.5) (end 141.1167 104.5901) (width 0.25) (layer "B.Cu") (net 4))
 (segment (start 127.5259 104.9458) (end 126.2116 106.2601) (width 0.25) (layer "F.Cu") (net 1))
 (segment (start 139.9845 104.9458) (end 127.5259 104.9458) (width 0.25) (layer "F.Cu") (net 1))
 (segment (start 126.2116 106.7577) (end 127.3652 107.9113) (width 0.25) (layer "F.Cu") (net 1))
 (segment (start 127.3652 107.9113) (end 128.125 107.9113) (width 0.25) (layer "F.Cu") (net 1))
 (segment (start 126.2116 106.2601) (end 126.2116 106.7577) (width 0.25) (layer "F.Cu") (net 1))
 (segment (start 128.125 108.7422) (end 128.125 107.9113) (width 0.25) (layer "F.Cu") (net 1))
 (via (at 139.9845 104.9458) (size 0.8) (drill 0.4) (layers "F.Cu" "B.Cu") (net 1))
 (segment (start 139.9845 102.803) (end 139.9845 104.9458) (width 0.25) (layer "B.Cu") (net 1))
 (segment (start 140.7875 102) (end 139.9845 102.803) (width 0.25) (layer "B.Cu") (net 1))
 (segment (start 142.2125 102) (end 140.7875 102) (width 0.25) (layer "B.Cu") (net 1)))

